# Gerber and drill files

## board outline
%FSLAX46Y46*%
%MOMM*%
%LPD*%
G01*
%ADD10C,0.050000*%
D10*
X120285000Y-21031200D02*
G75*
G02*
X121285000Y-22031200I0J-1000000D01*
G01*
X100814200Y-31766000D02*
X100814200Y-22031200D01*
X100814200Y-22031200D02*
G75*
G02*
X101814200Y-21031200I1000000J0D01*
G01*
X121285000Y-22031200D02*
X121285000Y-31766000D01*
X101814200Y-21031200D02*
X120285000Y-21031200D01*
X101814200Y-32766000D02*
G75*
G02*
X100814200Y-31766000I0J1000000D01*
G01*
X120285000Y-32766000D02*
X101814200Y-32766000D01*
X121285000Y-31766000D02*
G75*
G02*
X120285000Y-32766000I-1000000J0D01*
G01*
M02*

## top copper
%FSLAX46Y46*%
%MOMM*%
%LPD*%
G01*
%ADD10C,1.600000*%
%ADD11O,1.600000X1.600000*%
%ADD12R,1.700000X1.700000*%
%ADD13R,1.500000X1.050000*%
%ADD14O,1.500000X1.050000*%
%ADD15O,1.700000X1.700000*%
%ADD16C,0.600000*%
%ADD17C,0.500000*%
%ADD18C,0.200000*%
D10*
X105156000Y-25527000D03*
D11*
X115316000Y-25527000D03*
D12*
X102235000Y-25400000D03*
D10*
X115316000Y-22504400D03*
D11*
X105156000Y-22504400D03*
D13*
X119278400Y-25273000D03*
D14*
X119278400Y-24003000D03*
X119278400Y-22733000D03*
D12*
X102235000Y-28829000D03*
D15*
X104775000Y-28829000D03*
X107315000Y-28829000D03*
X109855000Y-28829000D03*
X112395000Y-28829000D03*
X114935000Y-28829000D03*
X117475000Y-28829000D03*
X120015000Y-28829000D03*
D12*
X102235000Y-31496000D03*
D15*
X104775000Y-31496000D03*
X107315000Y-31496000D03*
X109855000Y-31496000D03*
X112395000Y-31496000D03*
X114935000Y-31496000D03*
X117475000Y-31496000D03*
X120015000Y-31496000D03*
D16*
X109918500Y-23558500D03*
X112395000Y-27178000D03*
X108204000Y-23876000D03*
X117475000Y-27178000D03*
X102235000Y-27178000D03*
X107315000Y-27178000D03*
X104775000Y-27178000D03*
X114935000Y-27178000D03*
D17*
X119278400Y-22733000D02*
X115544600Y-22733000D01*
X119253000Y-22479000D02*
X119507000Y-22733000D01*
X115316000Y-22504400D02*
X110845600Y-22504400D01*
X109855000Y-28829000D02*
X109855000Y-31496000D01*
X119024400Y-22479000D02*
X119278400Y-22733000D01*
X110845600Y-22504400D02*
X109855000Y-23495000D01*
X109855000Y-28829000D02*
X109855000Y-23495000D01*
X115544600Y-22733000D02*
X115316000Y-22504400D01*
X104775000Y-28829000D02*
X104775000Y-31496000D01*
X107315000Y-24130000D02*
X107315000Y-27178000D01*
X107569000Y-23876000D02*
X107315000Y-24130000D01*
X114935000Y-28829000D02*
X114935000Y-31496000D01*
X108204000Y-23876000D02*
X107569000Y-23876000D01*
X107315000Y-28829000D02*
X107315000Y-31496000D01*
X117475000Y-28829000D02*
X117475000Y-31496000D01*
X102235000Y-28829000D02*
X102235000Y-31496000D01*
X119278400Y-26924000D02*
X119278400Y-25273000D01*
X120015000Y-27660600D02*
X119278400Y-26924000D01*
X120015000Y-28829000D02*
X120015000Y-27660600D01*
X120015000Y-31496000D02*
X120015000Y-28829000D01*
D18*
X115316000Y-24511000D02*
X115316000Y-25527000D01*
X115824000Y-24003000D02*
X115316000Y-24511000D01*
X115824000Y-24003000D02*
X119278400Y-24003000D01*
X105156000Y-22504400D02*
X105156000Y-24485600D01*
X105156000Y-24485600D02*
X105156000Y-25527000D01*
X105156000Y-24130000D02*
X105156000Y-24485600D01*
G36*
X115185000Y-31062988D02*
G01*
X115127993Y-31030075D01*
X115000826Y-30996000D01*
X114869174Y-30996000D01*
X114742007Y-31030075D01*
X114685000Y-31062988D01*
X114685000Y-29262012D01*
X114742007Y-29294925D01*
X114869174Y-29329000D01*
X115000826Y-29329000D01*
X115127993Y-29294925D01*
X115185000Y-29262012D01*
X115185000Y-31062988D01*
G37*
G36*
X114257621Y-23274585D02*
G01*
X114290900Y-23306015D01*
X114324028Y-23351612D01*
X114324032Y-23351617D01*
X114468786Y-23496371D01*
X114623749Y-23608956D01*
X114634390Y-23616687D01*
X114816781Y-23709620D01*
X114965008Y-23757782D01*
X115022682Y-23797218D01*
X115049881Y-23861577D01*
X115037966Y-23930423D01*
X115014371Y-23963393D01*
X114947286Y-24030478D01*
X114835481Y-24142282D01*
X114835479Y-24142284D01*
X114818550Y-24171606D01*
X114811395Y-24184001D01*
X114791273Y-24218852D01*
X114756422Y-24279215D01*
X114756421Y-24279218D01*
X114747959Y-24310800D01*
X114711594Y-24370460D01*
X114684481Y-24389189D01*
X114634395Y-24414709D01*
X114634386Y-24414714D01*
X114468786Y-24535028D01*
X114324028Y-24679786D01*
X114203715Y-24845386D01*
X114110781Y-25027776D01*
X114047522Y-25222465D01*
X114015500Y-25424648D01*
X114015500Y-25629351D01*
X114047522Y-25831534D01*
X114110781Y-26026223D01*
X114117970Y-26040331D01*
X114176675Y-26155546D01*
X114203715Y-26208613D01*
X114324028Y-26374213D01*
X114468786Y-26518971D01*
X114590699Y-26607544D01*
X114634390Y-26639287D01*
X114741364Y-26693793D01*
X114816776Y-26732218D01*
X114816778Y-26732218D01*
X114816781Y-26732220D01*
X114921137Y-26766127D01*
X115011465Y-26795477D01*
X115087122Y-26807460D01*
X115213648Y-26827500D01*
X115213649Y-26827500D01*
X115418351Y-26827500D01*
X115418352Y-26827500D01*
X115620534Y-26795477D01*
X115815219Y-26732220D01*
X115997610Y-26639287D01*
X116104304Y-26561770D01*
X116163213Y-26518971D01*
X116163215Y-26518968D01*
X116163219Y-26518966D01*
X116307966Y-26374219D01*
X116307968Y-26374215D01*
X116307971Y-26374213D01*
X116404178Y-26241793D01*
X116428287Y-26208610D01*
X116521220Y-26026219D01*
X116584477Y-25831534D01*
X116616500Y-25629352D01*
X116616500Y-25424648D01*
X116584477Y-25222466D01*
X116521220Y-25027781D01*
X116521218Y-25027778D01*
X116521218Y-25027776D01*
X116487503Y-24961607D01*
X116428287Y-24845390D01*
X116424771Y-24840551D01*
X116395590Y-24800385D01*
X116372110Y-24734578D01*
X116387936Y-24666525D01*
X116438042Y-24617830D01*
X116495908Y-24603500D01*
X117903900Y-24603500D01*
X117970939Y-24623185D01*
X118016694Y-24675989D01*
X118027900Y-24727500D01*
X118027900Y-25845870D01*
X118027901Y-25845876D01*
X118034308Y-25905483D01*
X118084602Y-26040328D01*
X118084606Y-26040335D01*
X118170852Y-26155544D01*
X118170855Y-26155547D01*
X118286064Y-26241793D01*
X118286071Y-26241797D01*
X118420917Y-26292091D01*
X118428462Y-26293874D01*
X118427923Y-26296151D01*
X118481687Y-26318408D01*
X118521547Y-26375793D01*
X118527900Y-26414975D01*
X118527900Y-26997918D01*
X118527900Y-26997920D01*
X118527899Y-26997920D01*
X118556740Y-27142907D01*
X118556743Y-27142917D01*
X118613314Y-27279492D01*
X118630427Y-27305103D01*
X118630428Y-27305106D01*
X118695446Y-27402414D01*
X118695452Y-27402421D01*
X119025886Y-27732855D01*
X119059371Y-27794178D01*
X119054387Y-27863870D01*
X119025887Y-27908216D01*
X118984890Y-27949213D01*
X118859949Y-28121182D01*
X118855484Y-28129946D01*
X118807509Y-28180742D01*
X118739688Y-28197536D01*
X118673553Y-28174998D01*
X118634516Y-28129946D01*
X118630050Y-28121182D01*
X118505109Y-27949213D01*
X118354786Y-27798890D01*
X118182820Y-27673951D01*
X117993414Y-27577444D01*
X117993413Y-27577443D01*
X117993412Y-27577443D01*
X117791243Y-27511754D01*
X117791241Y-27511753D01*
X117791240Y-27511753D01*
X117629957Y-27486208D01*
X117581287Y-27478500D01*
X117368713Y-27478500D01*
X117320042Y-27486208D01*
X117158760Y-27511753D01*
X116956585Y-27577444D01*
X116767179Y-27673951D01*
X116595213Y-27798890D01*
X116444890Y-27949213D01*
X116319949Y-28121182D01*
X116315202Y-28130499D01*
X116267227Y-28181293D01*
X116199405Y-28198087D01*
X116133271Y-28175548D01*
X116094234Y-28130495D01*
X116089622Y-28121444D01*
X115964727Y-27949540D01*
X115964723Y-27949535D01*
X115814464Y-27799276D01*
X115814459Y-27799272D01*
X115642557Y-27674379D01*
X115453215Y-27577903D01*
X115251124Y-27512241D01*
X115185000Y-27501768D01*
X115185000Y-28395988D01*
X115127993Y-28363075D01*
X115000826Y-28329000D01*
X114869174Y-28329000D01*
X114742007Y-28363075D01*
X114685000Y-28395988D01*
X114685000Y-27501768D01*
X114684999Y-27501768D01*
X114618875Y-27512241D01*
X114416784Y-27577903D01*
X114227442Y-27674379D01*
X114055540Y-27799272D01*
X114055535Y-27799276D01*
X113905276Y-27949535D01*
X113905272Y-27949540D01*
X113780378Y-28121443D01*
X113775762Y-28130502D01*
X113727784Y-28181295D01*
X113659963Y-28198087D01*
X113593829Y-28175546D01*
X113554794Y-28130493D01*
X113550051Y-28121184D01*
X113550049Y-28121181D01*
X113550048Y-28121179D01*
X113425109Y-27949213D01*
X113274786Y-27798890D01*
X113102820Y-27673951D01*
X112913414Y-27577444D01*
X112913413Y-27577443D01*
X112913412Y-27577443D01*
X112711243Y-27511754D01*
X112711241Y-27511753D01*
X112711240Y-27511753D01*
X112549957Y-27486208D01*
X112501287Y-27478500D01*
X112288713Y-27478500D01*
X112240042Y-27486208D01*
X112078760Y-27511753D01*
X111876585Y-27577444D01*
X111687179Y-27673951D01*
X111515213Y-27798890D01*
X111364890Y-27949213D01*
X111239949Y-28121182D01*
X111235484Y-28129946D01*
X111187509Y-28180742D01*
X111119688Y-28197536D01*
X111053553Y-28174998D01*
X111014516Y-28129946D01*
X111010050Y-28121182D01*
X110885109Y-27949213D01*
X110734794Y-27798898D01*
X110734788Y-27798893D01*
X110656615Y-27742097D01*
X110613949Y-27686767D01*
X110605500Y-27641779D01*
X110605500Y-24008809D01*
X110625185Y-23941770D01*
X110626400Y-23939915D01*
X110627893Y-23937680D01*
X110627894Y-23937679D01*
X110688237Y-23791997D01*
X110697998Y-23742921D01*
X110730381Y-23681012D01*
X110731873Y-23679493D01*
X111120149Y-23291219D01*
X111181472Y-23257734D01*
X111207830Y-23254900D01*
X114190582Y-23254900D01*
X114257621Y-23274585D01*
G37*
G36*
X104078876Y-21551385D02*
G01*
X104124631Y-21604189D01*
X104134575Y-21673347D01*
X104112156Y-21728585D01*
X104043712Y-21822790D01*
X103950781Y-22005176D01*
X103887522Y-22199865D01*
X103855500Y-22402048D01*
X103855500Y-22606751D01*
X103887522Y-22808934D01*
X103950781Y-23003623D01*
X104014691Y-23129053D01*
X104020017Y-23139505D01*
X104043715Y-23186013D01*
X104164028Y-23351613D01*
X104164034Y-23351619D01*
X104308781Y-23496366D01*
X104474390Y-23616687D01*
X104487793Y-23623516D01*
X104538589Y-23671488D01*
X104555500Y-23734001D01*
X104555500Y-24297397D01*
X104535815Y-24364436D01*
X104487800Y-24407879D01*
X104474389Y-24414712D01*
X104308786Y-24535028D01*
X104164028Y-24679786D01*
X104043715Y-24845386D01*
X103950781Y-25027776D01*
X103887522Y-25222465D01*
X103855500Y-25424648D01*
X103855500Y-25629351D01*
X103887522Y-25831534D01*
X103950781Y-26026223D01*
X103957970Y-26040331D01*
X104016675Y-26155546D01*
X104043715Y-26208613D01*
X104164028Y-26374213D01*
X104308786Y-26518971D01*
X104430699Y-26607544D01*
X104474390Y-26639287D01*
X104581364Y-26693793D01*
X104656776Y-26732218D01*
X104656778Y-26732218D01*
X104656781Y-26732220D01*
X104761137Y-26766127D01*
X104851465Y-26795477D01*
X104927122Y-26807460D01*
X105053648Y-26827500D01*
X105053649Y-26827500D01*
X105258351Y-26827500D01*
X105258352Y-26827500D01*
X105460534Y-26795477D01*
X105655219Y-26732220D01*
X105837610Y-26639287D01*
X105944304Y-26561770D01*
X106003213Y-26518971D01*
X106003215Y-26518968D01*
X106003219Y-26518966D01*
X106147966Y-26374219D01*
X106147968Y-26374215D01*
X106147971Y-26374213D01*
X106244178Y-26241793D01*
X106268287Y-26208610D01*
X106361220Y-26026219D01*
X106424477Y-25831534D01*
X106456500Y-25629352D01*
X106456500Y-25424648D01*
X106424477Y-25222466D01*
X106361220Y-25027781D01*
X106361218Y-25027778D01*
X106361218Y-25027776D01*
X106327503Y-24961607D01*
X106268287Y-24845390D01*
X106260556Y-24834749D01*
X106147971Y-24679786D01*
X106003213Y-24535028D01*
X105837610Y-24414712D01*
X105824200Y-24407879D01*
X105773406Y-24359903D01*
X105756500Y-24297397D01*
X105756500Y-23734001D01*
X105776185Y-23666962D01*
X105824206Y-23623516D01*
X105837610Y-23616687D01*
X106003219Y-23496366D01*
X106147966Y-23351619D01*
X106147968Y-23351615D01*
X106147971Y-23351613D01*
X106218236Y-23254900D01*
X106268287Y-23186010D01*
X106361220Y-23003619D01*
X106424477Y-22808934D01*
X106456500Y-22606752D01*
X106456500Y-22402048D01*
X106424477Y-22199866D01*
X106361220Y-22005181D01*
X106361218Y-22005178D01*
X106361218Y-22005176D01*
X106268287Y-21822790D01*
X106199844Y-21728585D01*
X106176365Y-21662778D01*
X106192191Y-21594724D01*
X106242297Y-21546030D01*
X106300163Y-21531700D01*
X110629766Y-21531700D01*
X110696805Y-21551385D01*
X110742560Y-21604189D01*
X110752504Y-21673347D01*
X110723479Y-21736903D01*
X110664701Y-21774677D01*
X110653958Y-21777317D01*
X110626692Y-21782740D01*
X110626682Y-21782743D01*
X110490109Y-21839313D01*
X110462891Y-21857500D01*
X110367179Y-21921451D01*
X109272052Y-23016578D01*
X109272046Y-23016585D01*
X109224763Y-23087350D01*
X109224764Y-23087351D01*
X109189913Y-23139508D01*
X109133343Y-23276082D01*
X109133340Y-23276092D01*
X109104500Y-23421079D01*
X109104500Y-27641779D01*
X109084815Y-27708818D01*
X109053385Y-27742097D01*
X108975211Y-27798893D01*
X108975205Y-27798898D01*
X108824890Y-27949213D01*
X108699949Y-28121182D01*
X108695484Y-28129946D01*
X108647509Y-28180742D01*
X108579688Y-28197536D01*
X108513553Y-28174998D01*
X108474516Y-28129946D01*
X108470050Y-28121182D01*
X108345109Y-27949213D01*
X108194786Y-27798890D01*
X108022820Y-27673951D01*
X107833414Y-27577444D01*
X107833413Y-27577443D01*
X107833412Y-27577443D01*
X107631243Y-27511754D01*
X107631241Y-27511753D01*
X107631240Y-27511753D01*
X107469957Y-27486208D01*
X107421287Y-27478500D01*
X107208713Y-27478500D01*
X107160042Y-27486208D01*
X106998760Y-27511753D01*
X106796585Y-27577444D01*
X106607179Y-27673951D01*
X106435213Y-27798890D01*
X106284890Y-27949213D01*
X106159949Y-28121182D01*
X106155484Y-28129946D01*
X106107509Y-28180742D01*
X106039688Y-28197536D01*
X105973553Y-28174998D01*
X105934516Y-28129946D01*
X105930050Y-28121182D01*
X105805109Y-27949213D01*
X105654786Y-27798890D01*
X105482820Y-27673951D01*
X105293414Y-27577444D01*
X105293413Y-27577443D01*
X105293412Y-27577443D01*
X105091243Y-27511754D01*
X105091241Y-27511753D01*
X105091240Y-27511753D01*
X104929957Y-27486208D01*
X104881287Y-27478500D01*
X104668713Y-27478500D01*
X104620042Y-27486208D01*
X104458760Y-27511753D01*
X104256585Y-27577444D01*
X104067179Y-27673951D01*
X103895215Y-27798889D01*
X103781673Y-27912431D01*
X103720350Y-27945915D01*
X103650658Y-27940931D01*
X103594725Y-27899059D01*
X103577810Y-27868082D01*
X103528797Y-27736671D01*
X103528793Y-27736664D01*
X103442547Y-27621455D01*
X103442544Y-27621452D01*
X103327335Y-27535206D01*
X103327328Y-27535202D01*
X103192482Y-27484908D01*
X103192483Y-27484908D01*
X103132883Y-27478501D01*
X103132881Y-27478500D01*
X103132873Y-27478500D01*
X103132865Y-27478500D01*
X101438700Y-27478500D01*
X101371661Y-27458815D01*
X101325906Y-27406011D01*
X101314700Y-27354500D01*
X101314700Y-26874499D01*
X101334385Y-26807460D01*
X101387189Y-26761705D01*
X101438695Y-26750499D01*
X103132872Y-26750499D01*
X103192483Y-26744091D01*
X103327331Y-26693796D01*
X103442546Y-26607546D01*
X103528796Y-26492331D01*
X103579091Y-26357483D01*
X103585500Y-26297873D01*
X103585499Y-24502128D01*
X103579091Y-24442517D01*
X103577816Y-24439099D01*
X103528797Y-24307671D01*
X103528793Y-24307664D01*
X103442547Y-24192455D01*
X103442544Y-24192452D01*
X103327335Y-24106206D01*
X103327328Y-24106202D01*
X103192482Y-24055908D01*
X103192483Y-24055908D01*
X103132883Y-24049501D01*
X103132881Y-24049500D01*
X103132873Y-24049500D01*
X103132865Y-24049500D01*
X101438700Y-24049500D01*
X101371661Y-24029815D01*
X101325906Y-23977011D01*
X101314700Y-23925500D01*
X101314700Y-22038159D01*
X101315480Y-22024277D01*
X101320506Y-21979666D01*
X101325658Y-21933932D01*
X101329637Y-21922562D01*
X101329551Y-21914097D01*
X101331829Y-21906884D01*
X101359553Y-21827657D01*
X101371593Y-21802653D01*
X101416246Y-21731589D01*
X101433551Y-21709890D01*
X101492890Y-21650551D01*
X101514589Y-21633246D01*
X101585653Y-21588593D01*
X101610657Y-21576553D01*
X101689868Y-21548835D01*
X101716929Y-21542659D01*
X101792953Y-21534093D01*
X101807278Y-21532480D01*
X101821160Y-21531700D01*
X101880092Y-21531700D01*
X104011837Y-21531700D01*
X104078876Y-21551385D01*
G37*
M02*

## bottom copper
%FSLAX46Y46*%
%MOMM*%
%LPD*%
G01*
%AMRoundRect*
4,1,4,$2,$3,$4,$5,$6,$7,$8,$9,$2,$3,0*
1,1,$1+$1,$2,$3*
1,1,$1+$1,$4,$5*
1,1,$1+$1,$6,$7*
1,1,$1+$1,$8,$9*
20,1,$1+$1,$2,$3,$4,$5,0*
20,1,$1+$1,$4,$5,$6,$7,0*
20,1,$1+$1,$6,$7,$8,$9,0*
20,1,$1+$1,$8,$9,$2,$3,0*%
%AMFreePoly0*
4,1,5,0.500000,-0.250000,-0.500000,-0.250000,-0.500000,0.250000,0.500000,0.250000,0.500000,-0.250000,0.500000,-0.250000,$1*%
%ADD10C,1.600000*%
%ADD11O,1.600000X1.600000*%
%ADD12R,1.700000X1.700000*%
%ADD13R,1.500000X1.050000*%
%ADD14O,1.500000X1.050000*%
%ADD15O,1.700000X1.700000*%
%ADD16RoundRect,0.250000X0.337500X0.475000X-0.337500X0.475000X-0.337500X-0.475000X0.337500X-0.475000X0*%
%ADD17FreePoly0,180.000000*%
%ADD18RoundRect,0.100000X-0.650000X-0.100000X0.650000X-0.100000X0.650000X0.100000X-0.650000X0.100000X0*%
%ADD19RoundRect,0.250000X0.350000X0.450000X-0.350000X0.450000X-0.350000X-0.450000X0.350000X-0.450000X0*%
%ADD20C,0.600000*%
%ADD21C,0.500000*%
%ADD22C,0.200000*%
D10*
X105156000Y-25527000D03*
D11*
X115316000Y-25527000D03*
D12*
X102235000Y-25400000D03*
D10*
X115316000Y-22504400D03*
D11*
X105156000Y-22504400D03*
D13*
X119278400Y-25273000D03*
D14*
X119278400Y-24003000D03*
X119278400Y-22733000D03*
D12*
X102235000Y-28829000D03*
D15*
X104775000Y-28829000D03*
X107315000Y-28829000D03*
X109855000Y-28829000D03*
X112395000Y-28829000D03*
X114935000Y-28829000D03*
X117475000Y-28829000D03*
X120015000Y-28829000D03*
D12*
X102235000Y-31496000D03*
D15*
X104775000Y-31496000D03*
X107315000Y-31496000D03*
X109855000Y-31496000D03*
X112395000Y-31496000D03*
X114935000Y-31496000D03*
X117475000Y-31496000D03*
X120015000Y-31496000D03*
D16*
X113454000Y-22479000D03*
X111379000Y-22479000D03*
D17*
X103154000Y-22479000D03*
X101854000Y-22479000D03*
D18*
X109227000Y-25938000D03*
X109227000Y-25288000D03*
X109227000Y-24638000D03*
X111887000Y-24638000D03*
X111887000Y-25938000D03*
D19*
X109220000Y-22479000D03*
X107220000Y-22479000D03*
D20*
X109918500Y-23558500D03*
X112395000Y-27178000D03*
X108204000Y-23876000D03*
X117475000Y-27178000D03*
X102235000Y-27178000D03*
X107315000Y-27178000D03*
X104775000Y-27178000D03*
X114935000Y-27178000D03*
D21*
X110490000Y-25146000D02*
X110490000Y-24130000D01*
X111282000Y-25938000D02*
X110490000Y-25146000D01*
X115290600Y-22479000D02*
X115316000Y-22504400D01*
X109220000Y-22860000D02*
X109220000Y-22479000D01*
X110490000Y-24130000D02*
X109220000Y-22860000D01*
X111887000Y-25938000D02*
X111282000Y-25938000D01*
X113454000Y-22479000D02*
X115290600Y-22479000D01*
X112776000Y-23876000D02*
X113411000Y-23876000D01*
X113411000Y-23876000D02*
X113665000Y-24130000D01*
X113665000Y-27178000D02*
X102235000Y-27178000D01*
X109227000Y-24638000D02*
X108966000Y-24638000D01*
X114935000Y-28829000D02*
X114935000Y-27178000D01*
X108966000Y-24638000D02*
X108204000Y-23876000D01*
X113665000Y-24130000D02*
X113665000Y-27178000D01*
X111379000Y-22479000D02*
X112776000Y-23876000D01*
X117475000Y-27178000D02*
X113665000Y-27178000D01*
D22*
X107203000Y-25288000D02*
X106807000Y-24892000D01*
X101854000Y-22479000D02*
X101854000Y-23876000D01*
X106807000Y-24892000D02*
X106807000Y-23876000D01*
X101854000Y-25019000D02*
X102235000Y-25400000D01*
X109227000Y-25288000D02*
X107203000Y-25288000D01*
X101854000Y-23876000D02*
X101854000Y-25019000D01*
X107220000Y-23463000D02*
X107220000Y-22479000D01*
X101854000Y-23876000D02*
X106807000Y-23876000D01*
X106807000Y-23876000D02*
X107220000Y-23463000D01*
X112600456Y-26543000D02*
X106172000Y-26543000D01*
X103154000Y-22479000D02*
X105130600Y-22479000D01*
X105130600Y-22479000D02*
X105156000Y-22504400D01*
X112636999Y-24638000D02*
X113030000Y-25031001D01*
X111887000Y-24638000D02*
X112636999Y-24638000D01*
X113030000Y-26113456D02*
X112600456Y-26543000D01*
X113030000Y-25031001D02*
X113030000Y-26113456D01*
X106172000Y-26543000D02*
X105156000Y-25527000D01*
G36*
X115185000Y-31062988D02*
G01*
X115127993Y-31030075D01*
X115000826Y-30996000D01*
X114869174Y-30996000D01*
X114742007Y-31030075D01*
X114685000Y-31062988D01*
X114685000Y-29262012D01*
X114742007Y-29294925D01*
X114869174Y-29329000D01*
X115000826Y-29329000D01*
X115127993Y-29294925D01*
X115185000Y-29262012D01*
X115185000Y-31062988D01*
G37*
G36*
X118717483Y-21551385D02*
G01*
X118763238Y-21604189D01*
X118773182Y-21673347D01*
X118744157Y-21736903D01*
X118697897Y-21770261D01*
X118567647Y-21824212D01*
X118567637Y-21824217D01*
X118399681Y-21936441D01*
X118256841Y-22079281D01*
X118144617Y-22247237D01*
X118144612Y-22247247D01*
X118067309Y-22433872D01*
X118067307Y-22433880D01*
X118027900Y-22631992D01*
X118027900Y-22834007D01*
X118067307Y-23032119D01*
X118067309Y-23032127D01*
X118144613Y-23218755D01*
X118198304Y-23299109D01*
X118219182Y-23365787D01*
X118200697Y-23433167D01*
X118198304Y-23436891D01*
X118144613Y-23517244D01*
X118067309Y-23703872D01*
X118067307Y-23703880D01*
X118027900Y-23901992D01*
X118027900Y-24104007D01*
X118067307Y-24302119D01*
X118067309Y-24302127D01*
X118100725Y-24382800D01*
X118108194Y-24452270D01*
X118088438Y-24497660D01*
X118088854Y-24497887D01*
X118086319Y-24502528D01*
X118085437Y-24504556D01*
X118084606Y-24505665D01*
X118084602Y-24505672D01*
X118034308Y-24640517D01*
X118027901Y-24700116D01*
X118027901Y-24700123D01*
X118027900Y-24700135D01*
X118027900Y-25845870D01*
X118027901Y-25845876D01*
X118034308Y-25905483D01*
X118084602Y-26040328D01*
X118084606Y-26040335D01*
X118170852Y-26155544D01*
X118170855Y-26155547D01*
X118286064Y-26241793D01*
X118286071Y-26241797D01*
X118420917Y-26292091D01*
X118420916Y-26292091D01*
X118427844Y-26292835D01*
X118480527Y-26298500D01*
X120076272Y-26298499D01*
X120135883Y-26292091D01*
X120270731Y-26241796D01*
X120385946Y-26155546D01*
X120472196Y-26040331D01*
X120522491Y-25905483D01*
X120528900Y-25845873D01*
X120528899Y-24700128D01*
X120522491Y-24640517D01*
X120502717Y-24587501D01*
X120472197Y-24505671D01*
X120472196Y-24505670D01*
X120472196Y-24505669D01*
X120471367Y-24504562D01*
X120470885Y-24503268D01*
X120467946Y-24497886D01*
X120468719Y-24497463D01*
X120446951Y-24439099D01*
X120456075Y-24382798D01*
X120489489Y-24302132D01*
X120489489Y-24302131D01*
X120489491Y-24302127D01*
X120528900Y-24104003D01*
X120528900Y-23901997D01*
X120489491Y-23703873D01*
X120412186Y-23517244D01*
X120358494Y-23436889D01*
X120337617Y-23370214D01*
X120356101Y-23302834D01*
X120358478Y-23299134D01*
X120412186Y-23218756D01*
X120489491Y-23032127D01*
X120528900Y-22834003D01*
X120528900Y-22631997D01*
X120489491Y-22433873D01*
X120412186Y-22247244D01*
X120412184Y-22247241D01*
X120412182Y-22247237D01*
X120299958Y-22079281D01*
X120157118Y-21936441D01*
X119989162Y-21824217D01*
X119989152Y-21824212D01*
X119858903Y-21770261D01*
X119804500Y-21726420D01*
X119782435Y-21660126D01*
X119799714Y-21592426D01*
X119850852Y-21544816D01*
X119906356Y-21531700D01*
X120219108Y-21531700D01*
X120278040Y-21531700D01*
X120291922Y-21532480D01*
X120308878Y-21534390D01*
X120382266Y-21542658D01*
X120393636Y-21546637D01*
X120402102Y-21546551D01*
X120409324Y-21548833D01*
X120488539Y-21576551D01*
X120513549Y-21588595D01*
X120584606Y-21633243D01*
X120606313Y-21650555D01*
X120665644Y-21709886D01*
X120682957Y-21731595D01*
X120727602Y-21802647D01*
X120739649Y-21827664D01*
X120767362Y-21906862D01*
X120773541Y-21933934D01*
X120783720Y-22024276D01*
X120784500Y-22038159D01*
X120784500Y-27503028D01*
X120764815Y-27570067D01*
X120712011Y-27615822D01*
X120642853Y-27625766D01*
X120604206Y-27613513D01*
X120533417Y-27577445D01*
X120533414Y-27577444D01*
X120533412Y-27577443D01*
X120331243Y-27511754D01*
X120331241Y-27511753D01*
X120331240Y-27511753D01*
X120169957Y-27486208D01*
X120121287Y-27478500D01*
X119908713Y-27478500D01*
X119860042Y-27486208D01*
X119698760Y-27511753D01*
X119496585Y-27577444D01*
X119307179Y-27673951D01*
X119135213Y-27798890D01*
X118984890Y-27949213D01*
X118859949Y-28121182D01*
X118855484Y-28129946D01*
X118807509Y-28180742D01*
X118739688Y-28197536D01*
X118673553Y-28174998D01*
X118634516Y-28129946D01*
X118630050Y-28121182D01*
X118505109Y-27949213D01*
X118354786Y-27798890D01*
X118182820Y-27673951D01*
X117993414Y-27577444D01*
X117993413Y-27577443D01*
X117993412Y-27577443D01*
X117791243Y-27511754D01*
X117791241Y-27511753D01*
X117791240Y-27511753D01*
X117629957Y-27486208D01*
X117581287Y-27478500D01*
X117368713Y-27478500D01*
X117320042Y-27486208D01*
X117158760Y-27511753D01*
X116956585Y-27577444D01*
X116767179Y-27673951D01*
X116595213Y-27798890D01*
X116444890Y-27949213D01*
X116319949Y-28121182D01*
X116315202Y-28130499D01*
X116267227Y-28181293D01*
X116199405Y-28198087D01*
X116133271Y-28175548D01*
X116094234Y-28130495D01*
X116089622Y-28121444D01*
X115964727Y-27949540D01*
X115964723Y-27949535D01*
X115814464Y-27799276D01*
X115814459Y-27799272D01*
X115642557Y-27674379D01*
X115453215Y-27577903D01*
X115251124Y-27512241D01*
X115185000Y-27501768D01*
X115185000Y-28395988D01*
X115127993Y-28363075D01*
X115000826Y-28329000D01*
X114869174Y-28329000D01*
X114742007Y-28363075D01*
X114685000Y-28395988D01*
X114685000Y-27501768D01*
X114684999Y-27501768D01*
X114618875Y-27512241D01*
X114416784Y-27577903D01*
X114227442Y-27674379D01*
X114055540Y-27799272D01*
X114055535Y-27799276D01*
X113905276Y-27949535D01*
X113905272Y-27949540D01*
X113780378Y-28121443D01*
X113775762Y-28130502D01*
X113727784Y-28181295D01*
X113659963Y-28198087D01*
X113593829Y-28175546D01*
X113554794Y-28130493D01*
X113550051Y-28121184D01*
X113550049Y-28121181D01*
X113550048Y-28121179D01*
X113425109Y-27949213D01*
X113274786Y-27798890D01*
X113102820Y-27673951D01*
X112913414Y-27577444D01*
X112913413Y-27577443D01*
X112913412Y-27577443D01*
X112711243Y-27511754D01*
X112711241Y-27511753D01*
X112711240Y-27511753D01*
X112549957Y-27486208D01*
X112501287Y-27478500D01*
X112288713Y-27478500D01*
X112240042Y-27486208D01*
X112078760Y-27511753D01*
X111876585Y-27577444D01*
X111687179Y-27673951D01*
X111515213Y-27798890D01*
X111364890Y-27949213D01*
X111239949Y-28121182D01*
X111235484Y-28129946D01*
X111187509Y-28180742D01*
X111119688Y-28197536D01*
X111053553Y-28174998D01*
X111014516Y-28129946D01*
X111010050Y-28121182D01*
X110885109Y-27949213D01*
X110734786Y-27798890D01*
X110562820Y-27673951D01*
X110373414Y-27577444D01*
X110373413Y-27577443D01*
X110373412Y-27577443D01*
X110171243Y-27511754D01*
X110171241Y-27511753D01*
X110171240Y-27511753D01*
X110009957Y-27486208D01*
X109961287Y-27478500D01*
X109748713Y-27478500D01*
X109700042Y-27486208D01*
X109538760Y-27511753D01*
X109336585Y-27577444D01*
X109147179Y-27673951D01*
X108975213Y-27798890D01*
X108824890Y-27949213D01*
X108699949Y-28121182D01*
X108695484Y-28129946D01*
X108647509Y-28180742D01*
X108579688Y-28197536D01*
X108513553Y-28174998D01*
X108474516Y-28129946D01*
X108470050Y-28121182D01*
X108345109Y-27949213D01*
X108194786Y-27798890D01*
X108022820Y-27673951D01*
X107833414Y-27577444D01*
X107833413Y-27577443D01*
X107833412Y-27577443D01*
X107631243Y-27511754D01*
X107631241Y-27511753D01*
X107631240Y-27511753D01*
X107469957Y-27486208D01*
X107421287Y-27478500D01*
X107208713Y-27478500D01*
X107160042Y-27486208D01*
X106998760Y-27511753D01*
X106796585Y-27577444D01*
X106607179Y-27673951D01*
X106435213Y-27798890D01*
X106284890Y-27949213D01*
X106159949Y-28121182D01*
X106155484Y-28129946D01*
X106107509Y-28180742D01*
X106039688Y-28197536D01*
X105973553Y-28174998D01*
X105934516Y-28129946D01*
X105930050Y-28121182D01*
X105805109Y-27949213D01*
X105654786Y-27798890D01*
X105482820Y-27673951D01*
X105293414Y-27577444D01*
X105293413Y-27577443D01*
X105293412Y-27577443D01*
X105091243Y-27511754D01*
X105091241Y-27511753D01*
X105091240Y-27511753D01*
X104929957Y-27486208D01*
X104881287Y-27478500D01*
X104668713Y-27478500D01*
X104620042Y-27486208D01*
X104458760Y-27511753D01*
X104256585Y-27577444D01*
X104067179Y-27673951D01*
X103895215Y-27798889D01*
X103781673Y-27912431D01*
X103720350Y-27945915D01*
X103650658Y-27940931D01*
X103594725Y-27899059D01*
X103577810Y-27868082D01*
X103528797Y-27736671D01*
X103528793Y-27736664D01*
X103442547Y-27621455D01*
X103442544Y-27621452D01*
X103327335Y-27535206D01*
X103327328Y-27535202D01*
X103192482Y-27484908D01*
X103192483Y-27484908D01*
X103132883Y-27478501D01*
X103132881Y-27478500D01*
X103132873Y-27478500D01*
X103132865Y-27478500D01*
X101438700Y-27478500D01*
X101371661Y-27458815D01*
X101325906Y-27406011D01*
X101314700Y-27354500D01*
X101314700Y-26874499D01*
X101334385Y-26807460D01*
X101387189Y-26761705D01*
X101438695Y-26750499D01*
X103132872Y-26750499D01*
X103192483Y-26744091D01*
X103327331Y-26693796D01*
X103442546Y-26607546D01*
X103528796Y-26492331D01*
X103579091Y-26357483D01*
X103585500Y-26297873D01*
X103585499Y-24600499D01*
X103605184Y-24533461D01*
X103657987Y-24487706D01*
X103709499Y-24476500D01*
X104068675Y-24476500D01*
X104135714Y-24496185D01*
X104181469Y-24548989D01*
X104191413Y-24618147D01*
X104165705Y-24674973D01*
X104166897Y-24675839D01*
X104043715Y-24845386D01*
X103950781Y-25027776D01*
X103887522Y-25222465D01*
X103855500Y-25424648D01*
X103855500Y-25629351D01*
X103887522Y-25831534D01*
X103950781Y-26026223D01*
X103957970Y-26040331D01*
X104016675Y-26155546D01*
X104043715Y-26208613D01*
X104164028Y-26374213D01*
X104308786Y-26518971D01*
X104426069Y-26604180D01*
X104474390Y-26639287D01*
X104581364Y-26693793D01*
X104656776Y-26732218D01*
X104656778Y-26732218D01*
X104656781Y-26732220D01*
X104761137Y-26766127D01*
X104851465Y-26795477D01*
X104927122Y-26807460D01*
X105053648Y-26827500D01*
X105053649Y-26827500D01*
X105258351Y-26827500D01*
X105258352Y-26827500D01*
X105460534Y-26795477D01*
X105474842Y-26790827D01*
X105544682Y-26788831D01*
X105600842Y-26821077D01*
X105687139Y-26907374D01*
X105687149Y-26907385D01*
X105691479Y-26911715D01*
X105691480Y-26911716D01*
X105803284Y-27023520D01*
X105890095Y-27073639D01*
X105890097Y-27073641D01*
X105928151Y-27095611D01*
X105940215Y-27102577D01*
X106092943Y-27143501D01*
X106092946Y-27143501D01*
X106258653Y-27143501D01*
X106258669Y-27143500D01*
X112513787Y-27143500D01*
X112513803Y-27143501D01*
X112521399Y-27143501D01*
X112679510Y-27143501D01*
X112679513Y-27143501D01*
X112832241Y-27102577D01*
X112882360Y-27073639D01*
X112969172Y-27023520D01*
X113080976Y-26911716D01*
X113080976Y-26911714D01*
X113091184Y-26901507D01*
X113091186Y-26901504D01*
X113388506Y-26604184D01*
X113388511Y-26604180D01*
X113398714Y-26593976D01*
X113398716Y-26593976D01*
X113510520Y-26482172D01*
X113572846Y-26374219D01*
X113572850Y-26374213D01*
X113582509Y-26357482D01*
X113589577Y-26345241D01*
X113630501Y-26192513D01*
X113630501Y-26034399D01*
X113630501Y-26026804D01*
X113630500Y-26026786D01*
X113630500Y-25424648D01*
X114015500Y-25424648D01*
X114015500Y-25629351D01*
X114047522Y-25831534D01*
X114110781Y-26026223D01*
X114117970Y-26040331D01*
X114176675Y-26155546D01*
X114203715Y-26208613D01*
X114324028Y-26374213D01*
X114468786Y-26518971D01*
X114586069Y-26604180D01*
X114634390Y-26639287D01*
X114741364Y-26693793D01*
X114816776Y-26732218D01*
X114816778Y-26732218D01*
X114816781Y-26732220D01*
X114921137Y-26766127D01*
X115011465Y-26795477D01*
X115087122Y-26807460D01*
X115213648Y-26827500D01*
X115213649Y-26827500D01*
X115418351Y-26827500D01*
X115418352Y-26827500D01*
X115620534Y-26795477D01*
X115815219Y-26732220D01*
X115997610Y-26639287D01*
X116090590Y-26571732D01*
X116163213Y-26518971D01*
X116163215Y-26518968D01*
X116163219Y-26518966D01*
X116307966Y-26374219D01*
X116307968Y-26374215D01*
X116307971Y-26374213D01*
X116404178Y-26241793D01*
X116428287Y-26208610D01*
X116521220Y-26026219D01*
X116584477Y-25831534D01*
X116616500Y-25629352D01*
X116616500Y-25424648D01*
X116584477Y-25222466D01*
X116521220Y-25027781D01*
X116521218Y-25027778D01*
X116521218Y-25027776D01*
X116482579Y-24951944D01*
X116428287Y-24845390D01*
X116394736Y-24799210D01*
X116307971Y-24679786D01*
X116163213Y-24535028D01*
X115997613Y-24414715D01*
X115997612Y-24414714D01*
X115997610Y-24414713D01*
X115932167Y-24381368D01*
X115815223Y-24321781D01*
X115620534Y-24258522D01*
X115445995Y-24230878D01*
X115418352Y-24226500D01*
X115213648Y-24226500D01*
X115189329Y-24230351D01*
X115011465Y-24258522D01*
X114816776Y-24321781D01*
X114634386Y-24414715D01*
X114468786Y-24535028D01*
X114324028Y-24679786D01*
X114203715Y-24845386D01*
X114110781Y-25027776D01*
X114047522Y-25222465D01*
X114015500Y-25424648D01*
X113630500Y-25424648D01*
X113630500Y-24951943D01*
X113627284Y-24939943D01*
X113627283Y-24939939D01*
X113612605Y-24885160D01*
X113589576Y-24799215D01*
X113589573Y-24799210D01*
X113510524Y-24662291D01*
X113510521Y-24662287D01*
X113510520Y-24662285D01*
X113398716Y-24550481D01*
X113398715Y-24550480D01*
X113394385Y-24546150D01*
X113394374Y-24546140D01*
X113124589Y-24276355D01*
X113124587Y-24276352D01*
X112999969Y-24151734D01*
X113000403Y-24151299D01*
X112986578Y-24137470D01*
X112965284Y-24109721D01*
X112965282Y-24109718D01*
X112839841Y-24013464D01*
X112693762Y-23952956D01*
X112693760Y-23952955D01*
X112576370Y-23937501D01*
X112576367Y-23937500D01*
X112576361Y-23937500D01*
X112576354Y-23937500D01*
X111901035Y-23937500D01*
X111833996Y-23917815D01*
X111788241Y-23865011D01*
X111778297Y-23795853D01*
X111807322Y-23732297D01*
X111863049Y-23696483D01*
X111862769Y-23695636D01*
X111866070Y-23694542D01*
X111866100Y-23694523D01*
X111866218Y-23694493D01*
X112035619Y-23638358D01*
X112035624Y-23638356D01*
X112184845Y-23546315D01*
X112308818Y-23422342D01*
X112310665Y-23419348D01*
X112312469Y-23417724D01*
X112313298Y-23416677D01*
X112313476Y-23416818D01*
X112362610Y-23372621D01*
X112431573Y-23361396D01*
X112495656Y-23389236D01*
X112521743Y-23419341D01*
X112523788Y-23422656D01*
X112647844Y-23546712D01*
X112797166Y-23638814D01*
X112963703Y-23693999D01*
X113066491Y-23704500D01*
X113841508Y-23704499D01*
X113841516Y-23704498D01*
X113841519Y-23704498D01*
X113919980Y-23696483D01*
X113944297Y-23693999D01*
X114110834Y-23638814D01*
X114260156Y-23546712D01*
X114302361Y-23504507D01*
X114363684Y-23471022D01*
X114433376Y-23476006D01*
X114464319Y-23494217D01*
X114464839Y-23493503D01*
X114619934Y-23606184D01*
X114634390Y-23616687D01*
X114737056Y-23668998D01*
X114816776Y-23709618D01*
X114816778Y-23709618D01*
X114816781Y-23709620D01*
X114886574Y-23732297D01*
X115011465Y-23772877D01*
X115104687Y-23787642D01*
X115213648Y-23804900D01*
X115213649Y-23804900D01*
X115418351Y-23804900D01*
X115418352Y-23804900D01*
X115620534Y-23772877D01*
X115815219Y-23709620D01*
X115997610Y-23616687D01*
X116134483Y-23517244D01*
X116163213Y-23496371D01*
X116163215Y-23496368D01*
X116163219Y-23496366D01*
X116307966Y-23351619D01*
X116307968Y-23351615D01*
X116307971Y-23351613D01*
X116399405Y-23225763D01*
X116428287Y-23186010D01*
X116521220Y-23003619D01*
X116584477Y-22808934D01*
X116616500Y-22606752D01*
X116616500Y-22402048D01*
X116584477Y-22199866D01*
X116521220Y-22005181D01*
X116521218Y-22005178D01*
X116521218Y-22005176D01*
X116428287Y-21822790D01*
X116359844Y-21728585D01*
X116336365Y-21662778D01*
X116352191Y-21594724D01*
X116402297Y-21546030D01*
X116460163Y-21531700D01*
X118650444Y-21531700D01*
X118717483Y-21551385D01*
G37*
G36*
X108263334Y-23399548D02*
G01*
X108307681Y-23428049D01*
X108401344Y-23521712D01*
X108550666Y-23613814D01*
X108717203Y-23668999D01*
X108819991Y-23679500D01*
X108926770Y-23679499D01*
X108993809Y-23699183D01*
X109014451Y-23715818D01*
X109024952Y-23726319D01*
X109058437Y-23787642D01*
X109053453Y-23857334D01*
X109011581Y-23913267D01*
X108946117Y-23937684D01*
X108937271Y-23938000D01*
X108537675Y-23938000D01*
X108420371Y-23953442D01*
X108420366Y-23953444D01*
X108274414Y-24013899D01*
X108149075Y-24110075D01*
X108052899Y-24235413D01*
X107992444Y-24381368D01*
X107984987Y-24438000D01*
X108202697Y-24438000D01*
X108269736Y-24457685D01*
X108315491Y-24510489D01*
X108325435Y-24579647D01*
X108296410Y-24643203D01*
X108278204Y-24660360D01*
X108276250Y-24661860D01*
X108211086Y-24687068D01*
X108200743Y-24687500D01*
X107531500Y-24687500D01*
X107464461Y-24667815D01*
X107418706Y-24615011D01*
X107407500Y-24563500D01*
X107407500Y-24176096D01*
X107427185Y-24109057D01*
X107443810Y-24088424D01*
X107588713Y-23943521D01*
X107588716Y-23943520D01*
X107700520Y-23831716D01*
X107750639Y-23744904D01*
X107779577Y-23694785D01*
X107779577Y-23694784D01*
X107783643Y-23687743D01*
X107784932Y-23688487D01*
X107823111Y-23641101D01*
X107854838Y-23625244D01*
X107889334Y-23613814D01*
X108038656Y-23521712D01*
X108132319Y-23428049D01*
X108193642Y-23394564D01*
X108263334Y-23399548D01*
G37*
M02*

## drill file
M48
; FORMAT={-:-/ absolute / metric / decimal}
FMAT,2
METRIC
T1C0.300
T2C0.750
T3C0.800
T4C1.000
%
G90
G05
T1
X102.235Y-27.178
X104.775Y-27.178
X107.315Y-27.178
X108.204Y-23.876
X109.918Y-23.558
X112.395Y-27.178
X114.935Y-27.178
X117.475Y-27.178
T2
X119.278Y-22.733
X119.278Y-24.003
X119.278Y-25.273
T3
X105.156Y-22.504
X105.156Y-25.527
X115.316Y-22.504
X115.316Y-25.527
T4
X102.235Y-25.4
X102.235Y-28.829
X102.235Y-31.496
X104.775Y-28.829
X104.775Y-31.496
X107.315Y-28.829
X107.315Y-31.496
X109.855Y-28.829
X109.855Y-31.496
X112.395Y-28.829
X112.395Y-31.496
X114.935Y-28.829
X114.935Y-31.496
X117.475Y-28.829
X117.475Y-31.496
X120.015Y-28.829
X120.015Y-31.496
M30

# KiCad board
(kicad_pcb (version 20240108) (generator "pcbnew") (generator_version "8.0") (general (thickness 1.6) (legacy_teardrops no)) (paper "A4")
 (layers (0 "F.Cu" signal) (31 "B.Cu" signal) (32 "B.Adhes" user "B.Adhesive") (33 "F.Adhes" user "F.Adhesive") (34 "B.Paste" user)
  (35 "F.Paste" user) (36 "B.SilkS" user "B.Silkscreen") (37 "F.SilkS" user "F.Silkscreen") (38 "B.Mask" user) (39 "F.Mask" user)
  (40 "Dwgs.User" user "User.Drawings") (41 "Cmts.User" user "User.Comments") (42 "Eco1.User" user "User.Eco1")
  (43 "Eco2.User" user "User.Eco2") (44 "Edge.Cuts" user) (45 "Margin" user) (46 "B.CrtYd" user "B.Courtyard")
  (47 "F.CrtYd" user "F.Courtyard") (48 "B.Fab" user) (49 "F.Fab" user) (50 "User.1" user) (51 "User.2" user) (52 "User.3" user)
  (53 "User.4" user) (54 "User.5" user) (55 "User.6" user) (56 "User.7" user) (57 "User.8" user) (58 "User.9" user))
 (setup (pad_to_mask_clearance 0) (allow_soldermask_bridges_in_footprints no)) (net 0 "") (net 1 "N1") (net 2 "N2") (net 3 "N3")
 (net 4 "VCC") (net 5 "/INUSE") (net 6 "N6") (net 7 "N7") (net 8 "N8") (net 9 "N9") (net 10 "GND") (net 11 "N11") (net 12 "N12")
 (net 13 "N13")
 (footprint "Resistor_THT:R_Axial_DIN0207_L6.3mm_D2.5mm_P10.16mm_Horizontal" (layer "F.Cu") (at 105.156 25.527)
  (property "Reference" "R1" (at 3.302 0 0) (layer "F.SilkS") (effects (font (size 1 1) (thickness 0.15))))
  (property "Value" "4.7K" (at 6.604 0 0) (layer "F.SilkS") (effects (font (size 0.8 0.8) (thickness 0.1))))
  (pad "1" thru_hole circle (at 0 0) (size 1.6 1.6) (drill 0.8) (layers "*.Cu" "*.Mask") (remove_unused_layers no) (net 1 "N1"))
  (pad "2" thru_hole oval (at 10.16 0) (size 1.6 1.6) (drill 0.8) (layers "*.Cu" "*.Mask") (remove_unused_layers no) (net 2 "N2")))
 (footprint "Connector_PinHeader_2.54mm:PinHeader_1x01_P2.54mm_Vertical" (layer "F.Cu") (at 102.235 25.4)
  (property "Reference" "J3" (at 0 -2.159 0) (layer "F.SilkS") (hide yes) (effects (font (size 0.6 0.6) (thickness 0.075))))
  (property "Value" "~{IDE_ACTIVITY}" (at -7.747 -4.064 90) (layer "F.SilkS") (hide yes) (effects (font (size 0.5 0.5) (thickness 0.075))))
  (pad "1" thru_hole rect (at 0 0) (size 1.7 1.7) (drill 1) (layers "*.Cu" "*.Mask") (remove_unused_layers no) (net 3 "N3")))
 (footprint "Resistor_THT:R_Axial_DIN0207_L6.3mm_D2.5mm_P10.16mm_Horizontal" (layer "F.Cu") (at 115.316 22.5044 180)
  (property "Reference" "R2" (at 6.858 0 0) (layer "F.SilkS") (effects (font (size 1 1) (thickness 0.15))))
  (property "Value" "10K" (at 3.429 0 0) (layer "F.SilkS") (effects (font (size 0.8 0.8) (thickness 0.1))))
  (pad "1" thru_hole circle (at 0 0 180) (size 1.6 1.6) (drill 0.8) (layers "*.Cu" "*.Mask") (remove_unused_layers no) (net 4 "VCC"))
  (pad "2" thru_hole oval (at 10.16 0 180) (size 1.6 1.6) (drill 0.8) (layers "*.Cu" "*.Mask") (remove_unused_layers no) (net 1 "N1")))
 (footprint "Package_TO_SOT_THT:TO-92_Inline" (layer "F.Cu") (at 119.2784 25.273 90)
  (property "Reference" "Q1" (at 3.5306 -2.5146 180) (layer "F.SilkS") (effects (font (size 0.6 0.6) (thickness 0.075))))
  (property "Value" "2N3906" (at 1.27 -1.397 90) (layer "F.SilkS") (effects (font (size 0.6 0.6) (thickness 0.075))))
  (pad "1" thru_hole rect (at 0 0 90) (size 1.05 1.5) (drill 0.75) (layers "*.Cu" "*.Mask") (remove_unused_layers no) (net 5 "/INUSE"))
  (pad "2" thru_hole oval (at 1.27 0 90) (size 1.05 1.5) (drill 0.75) (layers "*.Cu" "*.Mask") (remove_unused_layers no) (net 2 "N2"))
  (pad "3" thru_hole oval (at 2.54 0 90) (size 1.05 1.5) (drill 0.75) (layers "*.Cu" "*.Mask") (remove_unused_layers no) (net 4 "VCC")))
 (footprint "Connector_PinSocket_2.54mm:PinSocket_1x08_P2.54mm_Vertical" (layer "F.Cu") (at 102.235 28.829 90)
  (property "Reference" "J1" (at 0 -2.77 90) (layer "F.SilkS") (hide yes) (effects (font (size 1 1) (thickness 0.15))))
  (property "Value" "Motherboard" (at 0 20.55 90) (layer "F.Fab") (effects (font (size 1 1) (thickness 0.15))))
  (pad "1" thru_hole rect (at 0 0 90) (size 1.7 1.7) (drill 1) (layers "*.Cu" "*.Mask") (remove_unused_layers no) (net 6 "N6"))
  (pad "2" thru_hole oval (at 0 2.54 90) (size 1.7 1.7) (drill 1) (layers "*.Cu" "*.Mask") (remove_unused_layers no) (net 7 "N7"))
  (pad "3" thru_hole oval (at 0 5.08 90) (size 1.7 1.7) (drill 1) (layers "*.Cu" "*.Mask") (remove_unused_layers no) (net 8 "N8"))
  (pad "4" thru_hole oval (at 0 7.62 90) (size 1.7 1.7) (drill 1) (layers "*.Cu" "*.Mask") (remove_unused_layers no) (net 4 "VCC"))
  (pad "5" thru_hole oval (at 0 10.16 90) (size 1.7 1.7) (drill 1) (layers "*.Cu" "*.Mask") (remove_unused_layers no) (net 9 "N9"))
  (pad "6" thru_hole oval (at 0 12.7 90) (size 1.7 1.7) (drill 1) (layers "*.Cu" "*.Mask") (remove_unused_layers no) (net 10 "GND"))
  (pad "7" thru_hole oval (at 0 15.24 90) (size 1.7 1.7) (drill 1) (layers "*.Cu" "*.Mask") (remove_unused_layers no) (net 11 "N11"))
  (pad "8" thru_hole oval (at 0 17.78 90) (size 1.7 1.7) (drill 1) (layers "*.Cu" "*.Mask") (remove_unused_layers no) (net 5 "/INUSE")))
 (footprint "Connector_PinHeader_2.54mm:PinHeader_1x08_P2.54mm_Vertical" (layer "F.Cu") (at 102.235 31.496 90)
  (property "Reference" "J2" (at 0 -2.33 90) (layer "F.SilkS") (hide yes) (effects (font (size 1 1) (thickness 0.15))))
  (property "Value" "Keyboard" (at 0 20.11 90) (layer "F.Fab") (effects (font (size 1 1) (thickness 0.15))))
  (pad "1" thru_hole rect (at 0 0 90) (size 1.7 1.7) (drill 1) (layers "*.Cu" "*.Mask") (remove_unused_layers no) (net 6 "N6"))
  (pad "2" thru_hole oval (at 0 2.54 90) (size 1.7 1.7) (drill 1) (layers "*.Cu" "*.Mask") (remove_unused_layers no) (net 7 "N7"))
  (pad "3" thru_hole oval (at 0 5.08 90) (size 1.7 1.7) (drill 1) (layers "*.Cu" "*.Mask") (remove_unused_layers no) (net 8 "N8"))
  (pad "4" thru_hole oval (at 0 7.62 90) (size 1.7 1.7) (drill 1) (layers "*.Cu" "*.Mask") (remove_unused_layers no) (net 4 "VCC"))
  (pad "5" thru_hole oval (at 0 10.16 90) (size 1.7 1.7) (drill 1) (layers "*.Cu" "*.Mask") (remove_unused_layers no) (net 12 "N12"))
  (pad "6" thru_hole oval (at 0 12.7 90) (size 1.7 1.7) (drill 1) (layers "*.Cu" "*.Mask") (remove_unused_layers no) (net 10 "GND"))
  (pad "7" thru_hole oval (at 0 15.24 90) (size 1.7 1.7) (drill 1) (layers "*.Cu" "*.Mask") (remove_unused_layers no) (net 11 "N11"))
  (pad "8" thru_hole oval (at 0 17.78 90) (size 1.7 1.7) (drill 1) (layers "*.Cu" "*.Mask") (remove_unused_layers no) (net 5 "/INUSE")))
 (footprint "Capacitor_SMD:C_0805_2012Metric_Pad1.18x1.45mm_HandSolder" (layer "B.Cu") (at 112.4165 22.479 180)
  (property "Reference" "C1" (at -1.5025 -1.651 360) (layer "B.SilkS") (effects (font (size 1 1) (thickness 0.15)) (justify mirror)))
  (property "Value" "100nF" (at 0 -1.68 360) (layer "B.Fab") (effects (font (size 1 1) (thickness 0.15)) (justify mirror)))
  (pad "1" smd roundrect (at -1.0375 0 180) (size 1.175 1.45) (layers "B.Cu" "B.Paste" "B.Mask") (roundrect_rratio 0.212766) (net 4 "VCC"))
  (pad "2" smd roundrect (at 1.0375 0 180) (size 1.175 1.45) (layers "B.Cu" "B.Paste" "B.Mask") (roundrect_rratio 0.212766) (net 10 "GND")))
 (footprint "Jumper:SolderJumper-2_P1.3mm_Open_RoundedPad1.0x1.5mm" (layer "B.Cu") (at 102.504 22.479 180)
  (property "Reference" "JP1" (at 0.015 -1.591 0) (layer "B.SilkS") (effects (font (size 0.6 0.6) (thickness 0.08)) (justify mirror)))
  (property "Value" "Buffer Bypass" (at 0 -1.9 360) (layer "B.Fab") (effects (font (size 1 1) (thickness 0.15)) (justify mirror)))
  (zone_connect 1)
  (pad "1" smd custom (at -0.65 0 180) (size 1 0.5) (layers "B.Cu" "B.Mask") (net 1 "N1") (zone_connect 2) (thermal_bridge_angle 45)
   (options (clearance outline) (anchor rect)) (primitives))
  (pad "2" smd custom (at 0.65 0 180) (size 1 0.5) (layers "B.Cu" "B.Mask") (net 3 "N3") (zone_connect 2) (thermal_bridge_angle 45)
   (options (clearance outline) (anchor rect)) (primitives)))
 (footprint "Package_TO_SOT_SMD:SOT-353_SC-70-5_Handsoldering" (layer "B.Cu") (at 110.557 25.288)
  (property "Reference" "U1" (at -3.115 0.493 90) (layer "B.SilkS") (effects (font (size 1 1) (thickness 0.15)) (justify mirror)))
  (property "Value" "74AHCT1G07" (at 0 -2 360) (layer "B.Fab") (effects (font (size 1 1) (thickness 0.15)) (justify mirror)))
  (pad "1" smd roundrect (at -1.33 0.65) (size 1.5 0.4) (layers "B.Cu" "B.Paste" "B.Mask") (roundrect_rratio 0.25) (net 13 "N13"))
  (pad "2" smd roundrect (at -1.33 0) (size 1.5 0.4) (layers "B.Cu" "B.Paste" "B.Mask") (roundrect_rratio 0.25) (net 3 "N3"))
  (pad "3" smd roundrect (at -1.33 -0.65) (size 1.5 0.4) (layers "B.Cu" "B.Paste" "B.Mask") (roundrect_rratio 0.25) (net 10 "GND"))
  (pad "4" smd roundrect (at 1.33 -0.65) (size 1.5 0.4) (layers "B.Cu" "B.Paste" "B.Mask") (roundrect_rratio 0.25) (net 1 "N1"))
  (pad "5" smd roundrect (at 1.33 0.65) (size 1.5 0.4) (layers "B.Cu" "B.Paste" "B.Mask") (roundrect_rratio 0.25) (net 4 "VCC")))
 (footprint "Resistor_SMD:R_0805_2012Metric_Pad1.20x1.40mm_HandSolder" (layer "B.Cu") (at 108.22 22.479 180)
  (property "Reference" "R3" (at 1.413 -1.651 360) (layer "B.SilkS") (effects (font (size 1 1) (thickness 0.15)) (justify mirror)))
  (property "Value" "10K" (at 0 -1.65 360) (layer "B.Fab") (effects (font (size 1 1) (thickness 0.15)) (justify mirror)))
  (pad "1" smd roundrect (at -1 0 180) (size 1.2 1.4) (layers "B.Cu" "B.Paste" "B.Mask") (roundrect_rratio 0.208333) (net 4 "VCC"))
  (pad "2" smd roundrect (at 1 0 180) (size 1.2 1.4) (layers "B.Cu" "B.Paste" "B.Mask") (roundrect_rratio 0.208333) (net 3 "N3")))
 (gr_arc (start 120.285 21.0312) (mid 120.992107 21.324093) (end 121.285 22.0312) (stroke (width 0.05) (type default)) (layer "Edge.Cuts"))
 (gr_line (start 100.8142 31.766) (end 100.8142 22.0312) (stroke (width 0.05) (type default)) (layer "Edge.Cuts"))
 (gr_arc (start 100.8142 22.0312) (mid 101.107093 21.324093) (end 101.8142 21.0312) (stroke (width 0.05) (type default)) (layer "Edge.Cuts"))
 (gr_line (start 121.285 22.0312) (end 121.285 31.766) (stroke (width 0.05) (type default)) (layer "Edge.Cuts"))
 (gr_line (start 101.8142 21.0312) (end 120.285 21.0312) (stroke (width 0.05) (type default)) (layer "Edge.Cuts"))
 (gr_arc (start 101.8142 32.766) (mid 101.107093 32.473107) (end 100.8142 31.766) (stroke (width 0.05) (type default)) (layer "Edge.Cuts"))
 (gr_line (start 120.285 32.766) (end 101.8142 32.766) (stroke (width 0.05) (type default)) (layer "Edge.Cuts"))
 (gr_arc (start 121.285 31.766) (mid 120.992107 32.473107) (end 120.285 32.766) (stroke (width 0.05) (type default)) (layer "Edge.Cuts"))
 (segment (start 119.2784 22.733) (end 115.5446 22.733) (width 0.5) (layer "F.Cu") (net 4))
 (segment (start 119.253 22.479) (end 119.507 22.733) (width 0.5) (layer "F.Cu") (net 4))
 (segment (start 115.316 22.5044) (end 110.8456 22.5044) (width 0.5) (layer "F.Cu") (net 4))
 (segment (start 109.855 28.829) (end 109.855 31.496) (width 0.5) (layer "F.Cu") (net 4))
 (segment (start 119.0244 22.479) (end 119.2784 22.733) (width 0.5) (layer "F.Cu") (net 4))
 (segment (start 110.8456 22.5044) (end 109.855 23.495) (width 0.5) (layer "F.Cu") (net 4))
 (segment (start 109.855 28.829) (end 109.855 23.495) (width 0.5) (layer "F.Cu") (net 4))
 (segment (start 115.5446 22.733) (end 115.316 22.5044) (width 0.5) (layer "F.Cu") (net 4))
 (via (at 109.9185 23.5585) (size 0.6) (drill 0.3) (layers "F.Cu" "B.Cu") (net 4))
 (segment (start 110.49 25.146) (end 110.49 24.13) (width 0.5) (layer "B.Cu") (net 4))
 (segment (start 111.282 25.938) (end 110.49 25.146) (width 0.5) (layer "B.Cu") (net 4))
 (segment (start 115.2906 22.479) (end 115.316 22.5044) (width 0.5) (layer "B.Cu") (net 4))
 (segment (start 109.22 22.86) (end 109.22 22.479) (width 0.5) (layer "B.Cu") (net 4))
 (segment (start 110.49 24.13) (end 109.22 22.86) (width 0.5) (layer "B.Cu") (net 4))
 (segment (start 111.887 25.938) (end 111.282 25.938) (width 0.5) (layer "B.Cu") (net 4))
 (segment (start 113.454 22.479) (end 115.2906 22.479) (width 0.5) (layer "B.Cu") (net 4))
 (segment (start 104.775 28.829) (end 104.775 31.496) (width 0.5) (layer "F.Cu") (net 7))
 (segment (start 107.315 24.13) (end 107.315 27.178) (width 0.5) (layer "F.Cu") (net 10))
 (segment (start 107.569 23.876) (end 107.315 24.13) (width 0.5) (layer "F.Cu") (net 10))
 (segment (start 114.935 28.829) (end 114.935 31.496) (width 0.5) (layer "F.Cu") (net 10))
 (segment (start 108.204 23.876) (end 107.569 23.876) (width 0.5) (layer "F.Cu") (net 10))
 (via (at 112.395 27.178) (size 0.6) (drill 0.3) (layers "F.Cu" "B.Cu") (free yes) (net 10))
 (via (at 108.204 23.876) (size 0.6) (drill 0.3) (layers "F.Cu" "B.Cu") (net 10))
 (via (at 117.475 27.178) (size 0.6) (drill 0.3) (layers "F.Cu" "B.Cu") (free yes) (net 10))
 (via (at 102.235 27.178) (size 0.6) (drill 0.3) (layers "F.Cu" "B.Cu") (free yes) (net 10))
 (via (at 107.315 27.178) (size 0.6) (drill 0.3) (layers "F.Cu" "B.Cu") (free yes) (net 10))
 (via (at 104.775 27.178) (size 0.6) (drill 0.3) (layers "F.Cu" "B.Cu") (free yes) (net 10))
 (via (at 114.935 27.178) (size 0.6) (drill 0.3) (layers "F.Cu" "B.Cu") (free yes) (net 10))
 (segment (start 112.776 23.876) (end 113.411 23.876) (width 0.5) (layer "B.Cu") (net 10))
 (segment (start 113.411 23.876) (end 113.665 24.13) (width 0.5) (layer "B.Cu") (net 10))
 (segment (start 113.665 27.178) (end 102.235 27.178) (width 0.5) (layer "B.Cu") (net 10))
 (segment (start 109.227 24.638) (end 108.966 24.638) (width 0.5) (layer "B.Cu") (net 10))
 (segment (start 114.935 28.829) (end 114.935 27.178) (width 0.5) (layer "B.Cu") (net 10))
 (segment (start 108.966 24.638) (end 108.204 23.876) (width 0.5) (layer "B.Cu") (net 10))
 (segment (start 113.665 24.13) (end 113.665 27.178) (width 0.5) (layer "B.Cu") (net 10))
 (segment (start 111.379 22.479) (end 112.776 23.876) (width 0.5) (layer "B.Cu") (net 10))
 (segment (start 117.475 27.178) (end 113.665 27.178) (width 0.5) (layer "B.Cu") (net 10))
 (segment (start 107.315 28.829) (end 107.315 31.496) (width 0.5) (layer "F.Cu") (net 8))
 (segment (start 117.475 28.829) (end 117.475 31.496) (width 0.5) (layer "F.Cu") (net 11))
 (segment (start 102.235 28.829) (end 102.235 31.496) (width 0.5) (layer "F.Cu") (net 6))
 (segment (start 119.2784 26.924) (end 119.2784 25.273) (width 0.5) (layer "F.Cu") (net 5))
 (segment (start 120.015 27.6606) (end 119.2784 26.924) (width 0.5) (layer "F.Cu") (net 5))
 (segment (start 120.015 28.829) (end 120.015 27.6606) (width 0.5) (layer "F.Cu") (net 5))
 (segment (start 120.015 31.496) (end 120.015 28.829) (width 0.5) (layer "F.Cu") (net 5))
 (segment (start 107.203 25.288) (end 106.807 24.892) (width 0.2) (layer "B.Cu") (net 3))
 (segment (start 101.854 22.479) (end 101.854 23.876) (width 0.2) (layer "B.Cu") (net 3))
 (segment (start 106.807 24.892) (end 106.807 23.876) (width 0.2) (layer "B.Cu") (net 3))
 (segment (start 101.854 25.019) (end 102.235 25.4) (width 0.2) (layer "B.Cu") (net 3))
 (segment (start 109.227 25.288) (end 107.203 25.288) (width 0.2) (layer "B.Cu") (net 3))
 (segment (start 101.854 23.876) (end 101.854 25.019) (width 0.2) (layer "B.Cu") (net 3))
 (segment (start 107.22 23.463) (end 107.22 22.479) (width 0.2) (layer "B.Cu") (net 3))
 (segment (start 101.854 23.876) (end 106.807 23.876) (width 0.2) (layer "B.Cu") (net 3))
 (segment (start 106.807 23.876) (end 107.22 23.463) (width 0.2) (layer "B.Cu") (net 3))
 (segment (start 115.316 24.511) (end 115.316 25.527) (width 0.2) (layer "F.Cu") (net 2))
 (segment (start 115.824 24.003) (end 115.316 24.511) (width 0.2) (layer "F.Cu") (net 2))
 (segment (start 115.824 24.003) (end 119.2784 24.003) (width 0.2) (layer "F.Cu") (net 2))
 (segment (start 105.156 22.5044) (end 105.156 24.4856) (width 0.2) (layer "F.Cu") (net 1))
 (segment (start 105.156 24.4856) (end 105.156 25.527) (width 0.2) (layer "F.Cu") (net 1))
 (segment (start 105.156 24.13) (end 105.156 24.4856) (width 0.2) (layer "F.Cu") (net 1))
 (segment (start 112.600456 26.543) (end 106.172 26.543) (width 0.2) (layer "B.Cu") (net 1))
 (segment (start 103.154 22.479) (end 105.1306 22.479) (width 0.2) (layer "B.Cu") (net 1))
 (segment (start 105.1306 22.479) (end 105.156 22.5044) (width 0.2) (layer "B.Cu") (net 1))
 (segment (start 112.636999 24.638) (end 113.03 25.031001) (width 0.2) (layer "B.Cu") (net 1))
 (segment (start 111.887 24.638) (end 112.636999 24.638) (width 0.2) (layer "B.Cu") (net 1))
 (segment (start 113.03 26.113456) (end 112.600456 26.543) (width 0.2) (layer "B.Cu") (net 1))
 (segment (start 113.03 25.031001) (end 113.03 26.113456) (width 0.2) (layer "B.Cu") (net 1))
 (segment (start 106.172 26.543) (end 105.156 25.527) (width 0.2) (layer "B.Cu") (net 1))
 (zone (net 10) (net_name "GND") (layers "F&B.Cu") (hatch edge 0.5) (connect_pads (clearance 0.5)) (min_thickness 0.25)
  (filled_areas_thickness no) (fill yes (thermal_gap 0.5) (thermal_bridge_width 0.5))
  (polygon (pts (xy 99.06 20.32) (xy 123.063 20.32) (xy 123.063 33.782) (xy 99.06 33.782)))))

